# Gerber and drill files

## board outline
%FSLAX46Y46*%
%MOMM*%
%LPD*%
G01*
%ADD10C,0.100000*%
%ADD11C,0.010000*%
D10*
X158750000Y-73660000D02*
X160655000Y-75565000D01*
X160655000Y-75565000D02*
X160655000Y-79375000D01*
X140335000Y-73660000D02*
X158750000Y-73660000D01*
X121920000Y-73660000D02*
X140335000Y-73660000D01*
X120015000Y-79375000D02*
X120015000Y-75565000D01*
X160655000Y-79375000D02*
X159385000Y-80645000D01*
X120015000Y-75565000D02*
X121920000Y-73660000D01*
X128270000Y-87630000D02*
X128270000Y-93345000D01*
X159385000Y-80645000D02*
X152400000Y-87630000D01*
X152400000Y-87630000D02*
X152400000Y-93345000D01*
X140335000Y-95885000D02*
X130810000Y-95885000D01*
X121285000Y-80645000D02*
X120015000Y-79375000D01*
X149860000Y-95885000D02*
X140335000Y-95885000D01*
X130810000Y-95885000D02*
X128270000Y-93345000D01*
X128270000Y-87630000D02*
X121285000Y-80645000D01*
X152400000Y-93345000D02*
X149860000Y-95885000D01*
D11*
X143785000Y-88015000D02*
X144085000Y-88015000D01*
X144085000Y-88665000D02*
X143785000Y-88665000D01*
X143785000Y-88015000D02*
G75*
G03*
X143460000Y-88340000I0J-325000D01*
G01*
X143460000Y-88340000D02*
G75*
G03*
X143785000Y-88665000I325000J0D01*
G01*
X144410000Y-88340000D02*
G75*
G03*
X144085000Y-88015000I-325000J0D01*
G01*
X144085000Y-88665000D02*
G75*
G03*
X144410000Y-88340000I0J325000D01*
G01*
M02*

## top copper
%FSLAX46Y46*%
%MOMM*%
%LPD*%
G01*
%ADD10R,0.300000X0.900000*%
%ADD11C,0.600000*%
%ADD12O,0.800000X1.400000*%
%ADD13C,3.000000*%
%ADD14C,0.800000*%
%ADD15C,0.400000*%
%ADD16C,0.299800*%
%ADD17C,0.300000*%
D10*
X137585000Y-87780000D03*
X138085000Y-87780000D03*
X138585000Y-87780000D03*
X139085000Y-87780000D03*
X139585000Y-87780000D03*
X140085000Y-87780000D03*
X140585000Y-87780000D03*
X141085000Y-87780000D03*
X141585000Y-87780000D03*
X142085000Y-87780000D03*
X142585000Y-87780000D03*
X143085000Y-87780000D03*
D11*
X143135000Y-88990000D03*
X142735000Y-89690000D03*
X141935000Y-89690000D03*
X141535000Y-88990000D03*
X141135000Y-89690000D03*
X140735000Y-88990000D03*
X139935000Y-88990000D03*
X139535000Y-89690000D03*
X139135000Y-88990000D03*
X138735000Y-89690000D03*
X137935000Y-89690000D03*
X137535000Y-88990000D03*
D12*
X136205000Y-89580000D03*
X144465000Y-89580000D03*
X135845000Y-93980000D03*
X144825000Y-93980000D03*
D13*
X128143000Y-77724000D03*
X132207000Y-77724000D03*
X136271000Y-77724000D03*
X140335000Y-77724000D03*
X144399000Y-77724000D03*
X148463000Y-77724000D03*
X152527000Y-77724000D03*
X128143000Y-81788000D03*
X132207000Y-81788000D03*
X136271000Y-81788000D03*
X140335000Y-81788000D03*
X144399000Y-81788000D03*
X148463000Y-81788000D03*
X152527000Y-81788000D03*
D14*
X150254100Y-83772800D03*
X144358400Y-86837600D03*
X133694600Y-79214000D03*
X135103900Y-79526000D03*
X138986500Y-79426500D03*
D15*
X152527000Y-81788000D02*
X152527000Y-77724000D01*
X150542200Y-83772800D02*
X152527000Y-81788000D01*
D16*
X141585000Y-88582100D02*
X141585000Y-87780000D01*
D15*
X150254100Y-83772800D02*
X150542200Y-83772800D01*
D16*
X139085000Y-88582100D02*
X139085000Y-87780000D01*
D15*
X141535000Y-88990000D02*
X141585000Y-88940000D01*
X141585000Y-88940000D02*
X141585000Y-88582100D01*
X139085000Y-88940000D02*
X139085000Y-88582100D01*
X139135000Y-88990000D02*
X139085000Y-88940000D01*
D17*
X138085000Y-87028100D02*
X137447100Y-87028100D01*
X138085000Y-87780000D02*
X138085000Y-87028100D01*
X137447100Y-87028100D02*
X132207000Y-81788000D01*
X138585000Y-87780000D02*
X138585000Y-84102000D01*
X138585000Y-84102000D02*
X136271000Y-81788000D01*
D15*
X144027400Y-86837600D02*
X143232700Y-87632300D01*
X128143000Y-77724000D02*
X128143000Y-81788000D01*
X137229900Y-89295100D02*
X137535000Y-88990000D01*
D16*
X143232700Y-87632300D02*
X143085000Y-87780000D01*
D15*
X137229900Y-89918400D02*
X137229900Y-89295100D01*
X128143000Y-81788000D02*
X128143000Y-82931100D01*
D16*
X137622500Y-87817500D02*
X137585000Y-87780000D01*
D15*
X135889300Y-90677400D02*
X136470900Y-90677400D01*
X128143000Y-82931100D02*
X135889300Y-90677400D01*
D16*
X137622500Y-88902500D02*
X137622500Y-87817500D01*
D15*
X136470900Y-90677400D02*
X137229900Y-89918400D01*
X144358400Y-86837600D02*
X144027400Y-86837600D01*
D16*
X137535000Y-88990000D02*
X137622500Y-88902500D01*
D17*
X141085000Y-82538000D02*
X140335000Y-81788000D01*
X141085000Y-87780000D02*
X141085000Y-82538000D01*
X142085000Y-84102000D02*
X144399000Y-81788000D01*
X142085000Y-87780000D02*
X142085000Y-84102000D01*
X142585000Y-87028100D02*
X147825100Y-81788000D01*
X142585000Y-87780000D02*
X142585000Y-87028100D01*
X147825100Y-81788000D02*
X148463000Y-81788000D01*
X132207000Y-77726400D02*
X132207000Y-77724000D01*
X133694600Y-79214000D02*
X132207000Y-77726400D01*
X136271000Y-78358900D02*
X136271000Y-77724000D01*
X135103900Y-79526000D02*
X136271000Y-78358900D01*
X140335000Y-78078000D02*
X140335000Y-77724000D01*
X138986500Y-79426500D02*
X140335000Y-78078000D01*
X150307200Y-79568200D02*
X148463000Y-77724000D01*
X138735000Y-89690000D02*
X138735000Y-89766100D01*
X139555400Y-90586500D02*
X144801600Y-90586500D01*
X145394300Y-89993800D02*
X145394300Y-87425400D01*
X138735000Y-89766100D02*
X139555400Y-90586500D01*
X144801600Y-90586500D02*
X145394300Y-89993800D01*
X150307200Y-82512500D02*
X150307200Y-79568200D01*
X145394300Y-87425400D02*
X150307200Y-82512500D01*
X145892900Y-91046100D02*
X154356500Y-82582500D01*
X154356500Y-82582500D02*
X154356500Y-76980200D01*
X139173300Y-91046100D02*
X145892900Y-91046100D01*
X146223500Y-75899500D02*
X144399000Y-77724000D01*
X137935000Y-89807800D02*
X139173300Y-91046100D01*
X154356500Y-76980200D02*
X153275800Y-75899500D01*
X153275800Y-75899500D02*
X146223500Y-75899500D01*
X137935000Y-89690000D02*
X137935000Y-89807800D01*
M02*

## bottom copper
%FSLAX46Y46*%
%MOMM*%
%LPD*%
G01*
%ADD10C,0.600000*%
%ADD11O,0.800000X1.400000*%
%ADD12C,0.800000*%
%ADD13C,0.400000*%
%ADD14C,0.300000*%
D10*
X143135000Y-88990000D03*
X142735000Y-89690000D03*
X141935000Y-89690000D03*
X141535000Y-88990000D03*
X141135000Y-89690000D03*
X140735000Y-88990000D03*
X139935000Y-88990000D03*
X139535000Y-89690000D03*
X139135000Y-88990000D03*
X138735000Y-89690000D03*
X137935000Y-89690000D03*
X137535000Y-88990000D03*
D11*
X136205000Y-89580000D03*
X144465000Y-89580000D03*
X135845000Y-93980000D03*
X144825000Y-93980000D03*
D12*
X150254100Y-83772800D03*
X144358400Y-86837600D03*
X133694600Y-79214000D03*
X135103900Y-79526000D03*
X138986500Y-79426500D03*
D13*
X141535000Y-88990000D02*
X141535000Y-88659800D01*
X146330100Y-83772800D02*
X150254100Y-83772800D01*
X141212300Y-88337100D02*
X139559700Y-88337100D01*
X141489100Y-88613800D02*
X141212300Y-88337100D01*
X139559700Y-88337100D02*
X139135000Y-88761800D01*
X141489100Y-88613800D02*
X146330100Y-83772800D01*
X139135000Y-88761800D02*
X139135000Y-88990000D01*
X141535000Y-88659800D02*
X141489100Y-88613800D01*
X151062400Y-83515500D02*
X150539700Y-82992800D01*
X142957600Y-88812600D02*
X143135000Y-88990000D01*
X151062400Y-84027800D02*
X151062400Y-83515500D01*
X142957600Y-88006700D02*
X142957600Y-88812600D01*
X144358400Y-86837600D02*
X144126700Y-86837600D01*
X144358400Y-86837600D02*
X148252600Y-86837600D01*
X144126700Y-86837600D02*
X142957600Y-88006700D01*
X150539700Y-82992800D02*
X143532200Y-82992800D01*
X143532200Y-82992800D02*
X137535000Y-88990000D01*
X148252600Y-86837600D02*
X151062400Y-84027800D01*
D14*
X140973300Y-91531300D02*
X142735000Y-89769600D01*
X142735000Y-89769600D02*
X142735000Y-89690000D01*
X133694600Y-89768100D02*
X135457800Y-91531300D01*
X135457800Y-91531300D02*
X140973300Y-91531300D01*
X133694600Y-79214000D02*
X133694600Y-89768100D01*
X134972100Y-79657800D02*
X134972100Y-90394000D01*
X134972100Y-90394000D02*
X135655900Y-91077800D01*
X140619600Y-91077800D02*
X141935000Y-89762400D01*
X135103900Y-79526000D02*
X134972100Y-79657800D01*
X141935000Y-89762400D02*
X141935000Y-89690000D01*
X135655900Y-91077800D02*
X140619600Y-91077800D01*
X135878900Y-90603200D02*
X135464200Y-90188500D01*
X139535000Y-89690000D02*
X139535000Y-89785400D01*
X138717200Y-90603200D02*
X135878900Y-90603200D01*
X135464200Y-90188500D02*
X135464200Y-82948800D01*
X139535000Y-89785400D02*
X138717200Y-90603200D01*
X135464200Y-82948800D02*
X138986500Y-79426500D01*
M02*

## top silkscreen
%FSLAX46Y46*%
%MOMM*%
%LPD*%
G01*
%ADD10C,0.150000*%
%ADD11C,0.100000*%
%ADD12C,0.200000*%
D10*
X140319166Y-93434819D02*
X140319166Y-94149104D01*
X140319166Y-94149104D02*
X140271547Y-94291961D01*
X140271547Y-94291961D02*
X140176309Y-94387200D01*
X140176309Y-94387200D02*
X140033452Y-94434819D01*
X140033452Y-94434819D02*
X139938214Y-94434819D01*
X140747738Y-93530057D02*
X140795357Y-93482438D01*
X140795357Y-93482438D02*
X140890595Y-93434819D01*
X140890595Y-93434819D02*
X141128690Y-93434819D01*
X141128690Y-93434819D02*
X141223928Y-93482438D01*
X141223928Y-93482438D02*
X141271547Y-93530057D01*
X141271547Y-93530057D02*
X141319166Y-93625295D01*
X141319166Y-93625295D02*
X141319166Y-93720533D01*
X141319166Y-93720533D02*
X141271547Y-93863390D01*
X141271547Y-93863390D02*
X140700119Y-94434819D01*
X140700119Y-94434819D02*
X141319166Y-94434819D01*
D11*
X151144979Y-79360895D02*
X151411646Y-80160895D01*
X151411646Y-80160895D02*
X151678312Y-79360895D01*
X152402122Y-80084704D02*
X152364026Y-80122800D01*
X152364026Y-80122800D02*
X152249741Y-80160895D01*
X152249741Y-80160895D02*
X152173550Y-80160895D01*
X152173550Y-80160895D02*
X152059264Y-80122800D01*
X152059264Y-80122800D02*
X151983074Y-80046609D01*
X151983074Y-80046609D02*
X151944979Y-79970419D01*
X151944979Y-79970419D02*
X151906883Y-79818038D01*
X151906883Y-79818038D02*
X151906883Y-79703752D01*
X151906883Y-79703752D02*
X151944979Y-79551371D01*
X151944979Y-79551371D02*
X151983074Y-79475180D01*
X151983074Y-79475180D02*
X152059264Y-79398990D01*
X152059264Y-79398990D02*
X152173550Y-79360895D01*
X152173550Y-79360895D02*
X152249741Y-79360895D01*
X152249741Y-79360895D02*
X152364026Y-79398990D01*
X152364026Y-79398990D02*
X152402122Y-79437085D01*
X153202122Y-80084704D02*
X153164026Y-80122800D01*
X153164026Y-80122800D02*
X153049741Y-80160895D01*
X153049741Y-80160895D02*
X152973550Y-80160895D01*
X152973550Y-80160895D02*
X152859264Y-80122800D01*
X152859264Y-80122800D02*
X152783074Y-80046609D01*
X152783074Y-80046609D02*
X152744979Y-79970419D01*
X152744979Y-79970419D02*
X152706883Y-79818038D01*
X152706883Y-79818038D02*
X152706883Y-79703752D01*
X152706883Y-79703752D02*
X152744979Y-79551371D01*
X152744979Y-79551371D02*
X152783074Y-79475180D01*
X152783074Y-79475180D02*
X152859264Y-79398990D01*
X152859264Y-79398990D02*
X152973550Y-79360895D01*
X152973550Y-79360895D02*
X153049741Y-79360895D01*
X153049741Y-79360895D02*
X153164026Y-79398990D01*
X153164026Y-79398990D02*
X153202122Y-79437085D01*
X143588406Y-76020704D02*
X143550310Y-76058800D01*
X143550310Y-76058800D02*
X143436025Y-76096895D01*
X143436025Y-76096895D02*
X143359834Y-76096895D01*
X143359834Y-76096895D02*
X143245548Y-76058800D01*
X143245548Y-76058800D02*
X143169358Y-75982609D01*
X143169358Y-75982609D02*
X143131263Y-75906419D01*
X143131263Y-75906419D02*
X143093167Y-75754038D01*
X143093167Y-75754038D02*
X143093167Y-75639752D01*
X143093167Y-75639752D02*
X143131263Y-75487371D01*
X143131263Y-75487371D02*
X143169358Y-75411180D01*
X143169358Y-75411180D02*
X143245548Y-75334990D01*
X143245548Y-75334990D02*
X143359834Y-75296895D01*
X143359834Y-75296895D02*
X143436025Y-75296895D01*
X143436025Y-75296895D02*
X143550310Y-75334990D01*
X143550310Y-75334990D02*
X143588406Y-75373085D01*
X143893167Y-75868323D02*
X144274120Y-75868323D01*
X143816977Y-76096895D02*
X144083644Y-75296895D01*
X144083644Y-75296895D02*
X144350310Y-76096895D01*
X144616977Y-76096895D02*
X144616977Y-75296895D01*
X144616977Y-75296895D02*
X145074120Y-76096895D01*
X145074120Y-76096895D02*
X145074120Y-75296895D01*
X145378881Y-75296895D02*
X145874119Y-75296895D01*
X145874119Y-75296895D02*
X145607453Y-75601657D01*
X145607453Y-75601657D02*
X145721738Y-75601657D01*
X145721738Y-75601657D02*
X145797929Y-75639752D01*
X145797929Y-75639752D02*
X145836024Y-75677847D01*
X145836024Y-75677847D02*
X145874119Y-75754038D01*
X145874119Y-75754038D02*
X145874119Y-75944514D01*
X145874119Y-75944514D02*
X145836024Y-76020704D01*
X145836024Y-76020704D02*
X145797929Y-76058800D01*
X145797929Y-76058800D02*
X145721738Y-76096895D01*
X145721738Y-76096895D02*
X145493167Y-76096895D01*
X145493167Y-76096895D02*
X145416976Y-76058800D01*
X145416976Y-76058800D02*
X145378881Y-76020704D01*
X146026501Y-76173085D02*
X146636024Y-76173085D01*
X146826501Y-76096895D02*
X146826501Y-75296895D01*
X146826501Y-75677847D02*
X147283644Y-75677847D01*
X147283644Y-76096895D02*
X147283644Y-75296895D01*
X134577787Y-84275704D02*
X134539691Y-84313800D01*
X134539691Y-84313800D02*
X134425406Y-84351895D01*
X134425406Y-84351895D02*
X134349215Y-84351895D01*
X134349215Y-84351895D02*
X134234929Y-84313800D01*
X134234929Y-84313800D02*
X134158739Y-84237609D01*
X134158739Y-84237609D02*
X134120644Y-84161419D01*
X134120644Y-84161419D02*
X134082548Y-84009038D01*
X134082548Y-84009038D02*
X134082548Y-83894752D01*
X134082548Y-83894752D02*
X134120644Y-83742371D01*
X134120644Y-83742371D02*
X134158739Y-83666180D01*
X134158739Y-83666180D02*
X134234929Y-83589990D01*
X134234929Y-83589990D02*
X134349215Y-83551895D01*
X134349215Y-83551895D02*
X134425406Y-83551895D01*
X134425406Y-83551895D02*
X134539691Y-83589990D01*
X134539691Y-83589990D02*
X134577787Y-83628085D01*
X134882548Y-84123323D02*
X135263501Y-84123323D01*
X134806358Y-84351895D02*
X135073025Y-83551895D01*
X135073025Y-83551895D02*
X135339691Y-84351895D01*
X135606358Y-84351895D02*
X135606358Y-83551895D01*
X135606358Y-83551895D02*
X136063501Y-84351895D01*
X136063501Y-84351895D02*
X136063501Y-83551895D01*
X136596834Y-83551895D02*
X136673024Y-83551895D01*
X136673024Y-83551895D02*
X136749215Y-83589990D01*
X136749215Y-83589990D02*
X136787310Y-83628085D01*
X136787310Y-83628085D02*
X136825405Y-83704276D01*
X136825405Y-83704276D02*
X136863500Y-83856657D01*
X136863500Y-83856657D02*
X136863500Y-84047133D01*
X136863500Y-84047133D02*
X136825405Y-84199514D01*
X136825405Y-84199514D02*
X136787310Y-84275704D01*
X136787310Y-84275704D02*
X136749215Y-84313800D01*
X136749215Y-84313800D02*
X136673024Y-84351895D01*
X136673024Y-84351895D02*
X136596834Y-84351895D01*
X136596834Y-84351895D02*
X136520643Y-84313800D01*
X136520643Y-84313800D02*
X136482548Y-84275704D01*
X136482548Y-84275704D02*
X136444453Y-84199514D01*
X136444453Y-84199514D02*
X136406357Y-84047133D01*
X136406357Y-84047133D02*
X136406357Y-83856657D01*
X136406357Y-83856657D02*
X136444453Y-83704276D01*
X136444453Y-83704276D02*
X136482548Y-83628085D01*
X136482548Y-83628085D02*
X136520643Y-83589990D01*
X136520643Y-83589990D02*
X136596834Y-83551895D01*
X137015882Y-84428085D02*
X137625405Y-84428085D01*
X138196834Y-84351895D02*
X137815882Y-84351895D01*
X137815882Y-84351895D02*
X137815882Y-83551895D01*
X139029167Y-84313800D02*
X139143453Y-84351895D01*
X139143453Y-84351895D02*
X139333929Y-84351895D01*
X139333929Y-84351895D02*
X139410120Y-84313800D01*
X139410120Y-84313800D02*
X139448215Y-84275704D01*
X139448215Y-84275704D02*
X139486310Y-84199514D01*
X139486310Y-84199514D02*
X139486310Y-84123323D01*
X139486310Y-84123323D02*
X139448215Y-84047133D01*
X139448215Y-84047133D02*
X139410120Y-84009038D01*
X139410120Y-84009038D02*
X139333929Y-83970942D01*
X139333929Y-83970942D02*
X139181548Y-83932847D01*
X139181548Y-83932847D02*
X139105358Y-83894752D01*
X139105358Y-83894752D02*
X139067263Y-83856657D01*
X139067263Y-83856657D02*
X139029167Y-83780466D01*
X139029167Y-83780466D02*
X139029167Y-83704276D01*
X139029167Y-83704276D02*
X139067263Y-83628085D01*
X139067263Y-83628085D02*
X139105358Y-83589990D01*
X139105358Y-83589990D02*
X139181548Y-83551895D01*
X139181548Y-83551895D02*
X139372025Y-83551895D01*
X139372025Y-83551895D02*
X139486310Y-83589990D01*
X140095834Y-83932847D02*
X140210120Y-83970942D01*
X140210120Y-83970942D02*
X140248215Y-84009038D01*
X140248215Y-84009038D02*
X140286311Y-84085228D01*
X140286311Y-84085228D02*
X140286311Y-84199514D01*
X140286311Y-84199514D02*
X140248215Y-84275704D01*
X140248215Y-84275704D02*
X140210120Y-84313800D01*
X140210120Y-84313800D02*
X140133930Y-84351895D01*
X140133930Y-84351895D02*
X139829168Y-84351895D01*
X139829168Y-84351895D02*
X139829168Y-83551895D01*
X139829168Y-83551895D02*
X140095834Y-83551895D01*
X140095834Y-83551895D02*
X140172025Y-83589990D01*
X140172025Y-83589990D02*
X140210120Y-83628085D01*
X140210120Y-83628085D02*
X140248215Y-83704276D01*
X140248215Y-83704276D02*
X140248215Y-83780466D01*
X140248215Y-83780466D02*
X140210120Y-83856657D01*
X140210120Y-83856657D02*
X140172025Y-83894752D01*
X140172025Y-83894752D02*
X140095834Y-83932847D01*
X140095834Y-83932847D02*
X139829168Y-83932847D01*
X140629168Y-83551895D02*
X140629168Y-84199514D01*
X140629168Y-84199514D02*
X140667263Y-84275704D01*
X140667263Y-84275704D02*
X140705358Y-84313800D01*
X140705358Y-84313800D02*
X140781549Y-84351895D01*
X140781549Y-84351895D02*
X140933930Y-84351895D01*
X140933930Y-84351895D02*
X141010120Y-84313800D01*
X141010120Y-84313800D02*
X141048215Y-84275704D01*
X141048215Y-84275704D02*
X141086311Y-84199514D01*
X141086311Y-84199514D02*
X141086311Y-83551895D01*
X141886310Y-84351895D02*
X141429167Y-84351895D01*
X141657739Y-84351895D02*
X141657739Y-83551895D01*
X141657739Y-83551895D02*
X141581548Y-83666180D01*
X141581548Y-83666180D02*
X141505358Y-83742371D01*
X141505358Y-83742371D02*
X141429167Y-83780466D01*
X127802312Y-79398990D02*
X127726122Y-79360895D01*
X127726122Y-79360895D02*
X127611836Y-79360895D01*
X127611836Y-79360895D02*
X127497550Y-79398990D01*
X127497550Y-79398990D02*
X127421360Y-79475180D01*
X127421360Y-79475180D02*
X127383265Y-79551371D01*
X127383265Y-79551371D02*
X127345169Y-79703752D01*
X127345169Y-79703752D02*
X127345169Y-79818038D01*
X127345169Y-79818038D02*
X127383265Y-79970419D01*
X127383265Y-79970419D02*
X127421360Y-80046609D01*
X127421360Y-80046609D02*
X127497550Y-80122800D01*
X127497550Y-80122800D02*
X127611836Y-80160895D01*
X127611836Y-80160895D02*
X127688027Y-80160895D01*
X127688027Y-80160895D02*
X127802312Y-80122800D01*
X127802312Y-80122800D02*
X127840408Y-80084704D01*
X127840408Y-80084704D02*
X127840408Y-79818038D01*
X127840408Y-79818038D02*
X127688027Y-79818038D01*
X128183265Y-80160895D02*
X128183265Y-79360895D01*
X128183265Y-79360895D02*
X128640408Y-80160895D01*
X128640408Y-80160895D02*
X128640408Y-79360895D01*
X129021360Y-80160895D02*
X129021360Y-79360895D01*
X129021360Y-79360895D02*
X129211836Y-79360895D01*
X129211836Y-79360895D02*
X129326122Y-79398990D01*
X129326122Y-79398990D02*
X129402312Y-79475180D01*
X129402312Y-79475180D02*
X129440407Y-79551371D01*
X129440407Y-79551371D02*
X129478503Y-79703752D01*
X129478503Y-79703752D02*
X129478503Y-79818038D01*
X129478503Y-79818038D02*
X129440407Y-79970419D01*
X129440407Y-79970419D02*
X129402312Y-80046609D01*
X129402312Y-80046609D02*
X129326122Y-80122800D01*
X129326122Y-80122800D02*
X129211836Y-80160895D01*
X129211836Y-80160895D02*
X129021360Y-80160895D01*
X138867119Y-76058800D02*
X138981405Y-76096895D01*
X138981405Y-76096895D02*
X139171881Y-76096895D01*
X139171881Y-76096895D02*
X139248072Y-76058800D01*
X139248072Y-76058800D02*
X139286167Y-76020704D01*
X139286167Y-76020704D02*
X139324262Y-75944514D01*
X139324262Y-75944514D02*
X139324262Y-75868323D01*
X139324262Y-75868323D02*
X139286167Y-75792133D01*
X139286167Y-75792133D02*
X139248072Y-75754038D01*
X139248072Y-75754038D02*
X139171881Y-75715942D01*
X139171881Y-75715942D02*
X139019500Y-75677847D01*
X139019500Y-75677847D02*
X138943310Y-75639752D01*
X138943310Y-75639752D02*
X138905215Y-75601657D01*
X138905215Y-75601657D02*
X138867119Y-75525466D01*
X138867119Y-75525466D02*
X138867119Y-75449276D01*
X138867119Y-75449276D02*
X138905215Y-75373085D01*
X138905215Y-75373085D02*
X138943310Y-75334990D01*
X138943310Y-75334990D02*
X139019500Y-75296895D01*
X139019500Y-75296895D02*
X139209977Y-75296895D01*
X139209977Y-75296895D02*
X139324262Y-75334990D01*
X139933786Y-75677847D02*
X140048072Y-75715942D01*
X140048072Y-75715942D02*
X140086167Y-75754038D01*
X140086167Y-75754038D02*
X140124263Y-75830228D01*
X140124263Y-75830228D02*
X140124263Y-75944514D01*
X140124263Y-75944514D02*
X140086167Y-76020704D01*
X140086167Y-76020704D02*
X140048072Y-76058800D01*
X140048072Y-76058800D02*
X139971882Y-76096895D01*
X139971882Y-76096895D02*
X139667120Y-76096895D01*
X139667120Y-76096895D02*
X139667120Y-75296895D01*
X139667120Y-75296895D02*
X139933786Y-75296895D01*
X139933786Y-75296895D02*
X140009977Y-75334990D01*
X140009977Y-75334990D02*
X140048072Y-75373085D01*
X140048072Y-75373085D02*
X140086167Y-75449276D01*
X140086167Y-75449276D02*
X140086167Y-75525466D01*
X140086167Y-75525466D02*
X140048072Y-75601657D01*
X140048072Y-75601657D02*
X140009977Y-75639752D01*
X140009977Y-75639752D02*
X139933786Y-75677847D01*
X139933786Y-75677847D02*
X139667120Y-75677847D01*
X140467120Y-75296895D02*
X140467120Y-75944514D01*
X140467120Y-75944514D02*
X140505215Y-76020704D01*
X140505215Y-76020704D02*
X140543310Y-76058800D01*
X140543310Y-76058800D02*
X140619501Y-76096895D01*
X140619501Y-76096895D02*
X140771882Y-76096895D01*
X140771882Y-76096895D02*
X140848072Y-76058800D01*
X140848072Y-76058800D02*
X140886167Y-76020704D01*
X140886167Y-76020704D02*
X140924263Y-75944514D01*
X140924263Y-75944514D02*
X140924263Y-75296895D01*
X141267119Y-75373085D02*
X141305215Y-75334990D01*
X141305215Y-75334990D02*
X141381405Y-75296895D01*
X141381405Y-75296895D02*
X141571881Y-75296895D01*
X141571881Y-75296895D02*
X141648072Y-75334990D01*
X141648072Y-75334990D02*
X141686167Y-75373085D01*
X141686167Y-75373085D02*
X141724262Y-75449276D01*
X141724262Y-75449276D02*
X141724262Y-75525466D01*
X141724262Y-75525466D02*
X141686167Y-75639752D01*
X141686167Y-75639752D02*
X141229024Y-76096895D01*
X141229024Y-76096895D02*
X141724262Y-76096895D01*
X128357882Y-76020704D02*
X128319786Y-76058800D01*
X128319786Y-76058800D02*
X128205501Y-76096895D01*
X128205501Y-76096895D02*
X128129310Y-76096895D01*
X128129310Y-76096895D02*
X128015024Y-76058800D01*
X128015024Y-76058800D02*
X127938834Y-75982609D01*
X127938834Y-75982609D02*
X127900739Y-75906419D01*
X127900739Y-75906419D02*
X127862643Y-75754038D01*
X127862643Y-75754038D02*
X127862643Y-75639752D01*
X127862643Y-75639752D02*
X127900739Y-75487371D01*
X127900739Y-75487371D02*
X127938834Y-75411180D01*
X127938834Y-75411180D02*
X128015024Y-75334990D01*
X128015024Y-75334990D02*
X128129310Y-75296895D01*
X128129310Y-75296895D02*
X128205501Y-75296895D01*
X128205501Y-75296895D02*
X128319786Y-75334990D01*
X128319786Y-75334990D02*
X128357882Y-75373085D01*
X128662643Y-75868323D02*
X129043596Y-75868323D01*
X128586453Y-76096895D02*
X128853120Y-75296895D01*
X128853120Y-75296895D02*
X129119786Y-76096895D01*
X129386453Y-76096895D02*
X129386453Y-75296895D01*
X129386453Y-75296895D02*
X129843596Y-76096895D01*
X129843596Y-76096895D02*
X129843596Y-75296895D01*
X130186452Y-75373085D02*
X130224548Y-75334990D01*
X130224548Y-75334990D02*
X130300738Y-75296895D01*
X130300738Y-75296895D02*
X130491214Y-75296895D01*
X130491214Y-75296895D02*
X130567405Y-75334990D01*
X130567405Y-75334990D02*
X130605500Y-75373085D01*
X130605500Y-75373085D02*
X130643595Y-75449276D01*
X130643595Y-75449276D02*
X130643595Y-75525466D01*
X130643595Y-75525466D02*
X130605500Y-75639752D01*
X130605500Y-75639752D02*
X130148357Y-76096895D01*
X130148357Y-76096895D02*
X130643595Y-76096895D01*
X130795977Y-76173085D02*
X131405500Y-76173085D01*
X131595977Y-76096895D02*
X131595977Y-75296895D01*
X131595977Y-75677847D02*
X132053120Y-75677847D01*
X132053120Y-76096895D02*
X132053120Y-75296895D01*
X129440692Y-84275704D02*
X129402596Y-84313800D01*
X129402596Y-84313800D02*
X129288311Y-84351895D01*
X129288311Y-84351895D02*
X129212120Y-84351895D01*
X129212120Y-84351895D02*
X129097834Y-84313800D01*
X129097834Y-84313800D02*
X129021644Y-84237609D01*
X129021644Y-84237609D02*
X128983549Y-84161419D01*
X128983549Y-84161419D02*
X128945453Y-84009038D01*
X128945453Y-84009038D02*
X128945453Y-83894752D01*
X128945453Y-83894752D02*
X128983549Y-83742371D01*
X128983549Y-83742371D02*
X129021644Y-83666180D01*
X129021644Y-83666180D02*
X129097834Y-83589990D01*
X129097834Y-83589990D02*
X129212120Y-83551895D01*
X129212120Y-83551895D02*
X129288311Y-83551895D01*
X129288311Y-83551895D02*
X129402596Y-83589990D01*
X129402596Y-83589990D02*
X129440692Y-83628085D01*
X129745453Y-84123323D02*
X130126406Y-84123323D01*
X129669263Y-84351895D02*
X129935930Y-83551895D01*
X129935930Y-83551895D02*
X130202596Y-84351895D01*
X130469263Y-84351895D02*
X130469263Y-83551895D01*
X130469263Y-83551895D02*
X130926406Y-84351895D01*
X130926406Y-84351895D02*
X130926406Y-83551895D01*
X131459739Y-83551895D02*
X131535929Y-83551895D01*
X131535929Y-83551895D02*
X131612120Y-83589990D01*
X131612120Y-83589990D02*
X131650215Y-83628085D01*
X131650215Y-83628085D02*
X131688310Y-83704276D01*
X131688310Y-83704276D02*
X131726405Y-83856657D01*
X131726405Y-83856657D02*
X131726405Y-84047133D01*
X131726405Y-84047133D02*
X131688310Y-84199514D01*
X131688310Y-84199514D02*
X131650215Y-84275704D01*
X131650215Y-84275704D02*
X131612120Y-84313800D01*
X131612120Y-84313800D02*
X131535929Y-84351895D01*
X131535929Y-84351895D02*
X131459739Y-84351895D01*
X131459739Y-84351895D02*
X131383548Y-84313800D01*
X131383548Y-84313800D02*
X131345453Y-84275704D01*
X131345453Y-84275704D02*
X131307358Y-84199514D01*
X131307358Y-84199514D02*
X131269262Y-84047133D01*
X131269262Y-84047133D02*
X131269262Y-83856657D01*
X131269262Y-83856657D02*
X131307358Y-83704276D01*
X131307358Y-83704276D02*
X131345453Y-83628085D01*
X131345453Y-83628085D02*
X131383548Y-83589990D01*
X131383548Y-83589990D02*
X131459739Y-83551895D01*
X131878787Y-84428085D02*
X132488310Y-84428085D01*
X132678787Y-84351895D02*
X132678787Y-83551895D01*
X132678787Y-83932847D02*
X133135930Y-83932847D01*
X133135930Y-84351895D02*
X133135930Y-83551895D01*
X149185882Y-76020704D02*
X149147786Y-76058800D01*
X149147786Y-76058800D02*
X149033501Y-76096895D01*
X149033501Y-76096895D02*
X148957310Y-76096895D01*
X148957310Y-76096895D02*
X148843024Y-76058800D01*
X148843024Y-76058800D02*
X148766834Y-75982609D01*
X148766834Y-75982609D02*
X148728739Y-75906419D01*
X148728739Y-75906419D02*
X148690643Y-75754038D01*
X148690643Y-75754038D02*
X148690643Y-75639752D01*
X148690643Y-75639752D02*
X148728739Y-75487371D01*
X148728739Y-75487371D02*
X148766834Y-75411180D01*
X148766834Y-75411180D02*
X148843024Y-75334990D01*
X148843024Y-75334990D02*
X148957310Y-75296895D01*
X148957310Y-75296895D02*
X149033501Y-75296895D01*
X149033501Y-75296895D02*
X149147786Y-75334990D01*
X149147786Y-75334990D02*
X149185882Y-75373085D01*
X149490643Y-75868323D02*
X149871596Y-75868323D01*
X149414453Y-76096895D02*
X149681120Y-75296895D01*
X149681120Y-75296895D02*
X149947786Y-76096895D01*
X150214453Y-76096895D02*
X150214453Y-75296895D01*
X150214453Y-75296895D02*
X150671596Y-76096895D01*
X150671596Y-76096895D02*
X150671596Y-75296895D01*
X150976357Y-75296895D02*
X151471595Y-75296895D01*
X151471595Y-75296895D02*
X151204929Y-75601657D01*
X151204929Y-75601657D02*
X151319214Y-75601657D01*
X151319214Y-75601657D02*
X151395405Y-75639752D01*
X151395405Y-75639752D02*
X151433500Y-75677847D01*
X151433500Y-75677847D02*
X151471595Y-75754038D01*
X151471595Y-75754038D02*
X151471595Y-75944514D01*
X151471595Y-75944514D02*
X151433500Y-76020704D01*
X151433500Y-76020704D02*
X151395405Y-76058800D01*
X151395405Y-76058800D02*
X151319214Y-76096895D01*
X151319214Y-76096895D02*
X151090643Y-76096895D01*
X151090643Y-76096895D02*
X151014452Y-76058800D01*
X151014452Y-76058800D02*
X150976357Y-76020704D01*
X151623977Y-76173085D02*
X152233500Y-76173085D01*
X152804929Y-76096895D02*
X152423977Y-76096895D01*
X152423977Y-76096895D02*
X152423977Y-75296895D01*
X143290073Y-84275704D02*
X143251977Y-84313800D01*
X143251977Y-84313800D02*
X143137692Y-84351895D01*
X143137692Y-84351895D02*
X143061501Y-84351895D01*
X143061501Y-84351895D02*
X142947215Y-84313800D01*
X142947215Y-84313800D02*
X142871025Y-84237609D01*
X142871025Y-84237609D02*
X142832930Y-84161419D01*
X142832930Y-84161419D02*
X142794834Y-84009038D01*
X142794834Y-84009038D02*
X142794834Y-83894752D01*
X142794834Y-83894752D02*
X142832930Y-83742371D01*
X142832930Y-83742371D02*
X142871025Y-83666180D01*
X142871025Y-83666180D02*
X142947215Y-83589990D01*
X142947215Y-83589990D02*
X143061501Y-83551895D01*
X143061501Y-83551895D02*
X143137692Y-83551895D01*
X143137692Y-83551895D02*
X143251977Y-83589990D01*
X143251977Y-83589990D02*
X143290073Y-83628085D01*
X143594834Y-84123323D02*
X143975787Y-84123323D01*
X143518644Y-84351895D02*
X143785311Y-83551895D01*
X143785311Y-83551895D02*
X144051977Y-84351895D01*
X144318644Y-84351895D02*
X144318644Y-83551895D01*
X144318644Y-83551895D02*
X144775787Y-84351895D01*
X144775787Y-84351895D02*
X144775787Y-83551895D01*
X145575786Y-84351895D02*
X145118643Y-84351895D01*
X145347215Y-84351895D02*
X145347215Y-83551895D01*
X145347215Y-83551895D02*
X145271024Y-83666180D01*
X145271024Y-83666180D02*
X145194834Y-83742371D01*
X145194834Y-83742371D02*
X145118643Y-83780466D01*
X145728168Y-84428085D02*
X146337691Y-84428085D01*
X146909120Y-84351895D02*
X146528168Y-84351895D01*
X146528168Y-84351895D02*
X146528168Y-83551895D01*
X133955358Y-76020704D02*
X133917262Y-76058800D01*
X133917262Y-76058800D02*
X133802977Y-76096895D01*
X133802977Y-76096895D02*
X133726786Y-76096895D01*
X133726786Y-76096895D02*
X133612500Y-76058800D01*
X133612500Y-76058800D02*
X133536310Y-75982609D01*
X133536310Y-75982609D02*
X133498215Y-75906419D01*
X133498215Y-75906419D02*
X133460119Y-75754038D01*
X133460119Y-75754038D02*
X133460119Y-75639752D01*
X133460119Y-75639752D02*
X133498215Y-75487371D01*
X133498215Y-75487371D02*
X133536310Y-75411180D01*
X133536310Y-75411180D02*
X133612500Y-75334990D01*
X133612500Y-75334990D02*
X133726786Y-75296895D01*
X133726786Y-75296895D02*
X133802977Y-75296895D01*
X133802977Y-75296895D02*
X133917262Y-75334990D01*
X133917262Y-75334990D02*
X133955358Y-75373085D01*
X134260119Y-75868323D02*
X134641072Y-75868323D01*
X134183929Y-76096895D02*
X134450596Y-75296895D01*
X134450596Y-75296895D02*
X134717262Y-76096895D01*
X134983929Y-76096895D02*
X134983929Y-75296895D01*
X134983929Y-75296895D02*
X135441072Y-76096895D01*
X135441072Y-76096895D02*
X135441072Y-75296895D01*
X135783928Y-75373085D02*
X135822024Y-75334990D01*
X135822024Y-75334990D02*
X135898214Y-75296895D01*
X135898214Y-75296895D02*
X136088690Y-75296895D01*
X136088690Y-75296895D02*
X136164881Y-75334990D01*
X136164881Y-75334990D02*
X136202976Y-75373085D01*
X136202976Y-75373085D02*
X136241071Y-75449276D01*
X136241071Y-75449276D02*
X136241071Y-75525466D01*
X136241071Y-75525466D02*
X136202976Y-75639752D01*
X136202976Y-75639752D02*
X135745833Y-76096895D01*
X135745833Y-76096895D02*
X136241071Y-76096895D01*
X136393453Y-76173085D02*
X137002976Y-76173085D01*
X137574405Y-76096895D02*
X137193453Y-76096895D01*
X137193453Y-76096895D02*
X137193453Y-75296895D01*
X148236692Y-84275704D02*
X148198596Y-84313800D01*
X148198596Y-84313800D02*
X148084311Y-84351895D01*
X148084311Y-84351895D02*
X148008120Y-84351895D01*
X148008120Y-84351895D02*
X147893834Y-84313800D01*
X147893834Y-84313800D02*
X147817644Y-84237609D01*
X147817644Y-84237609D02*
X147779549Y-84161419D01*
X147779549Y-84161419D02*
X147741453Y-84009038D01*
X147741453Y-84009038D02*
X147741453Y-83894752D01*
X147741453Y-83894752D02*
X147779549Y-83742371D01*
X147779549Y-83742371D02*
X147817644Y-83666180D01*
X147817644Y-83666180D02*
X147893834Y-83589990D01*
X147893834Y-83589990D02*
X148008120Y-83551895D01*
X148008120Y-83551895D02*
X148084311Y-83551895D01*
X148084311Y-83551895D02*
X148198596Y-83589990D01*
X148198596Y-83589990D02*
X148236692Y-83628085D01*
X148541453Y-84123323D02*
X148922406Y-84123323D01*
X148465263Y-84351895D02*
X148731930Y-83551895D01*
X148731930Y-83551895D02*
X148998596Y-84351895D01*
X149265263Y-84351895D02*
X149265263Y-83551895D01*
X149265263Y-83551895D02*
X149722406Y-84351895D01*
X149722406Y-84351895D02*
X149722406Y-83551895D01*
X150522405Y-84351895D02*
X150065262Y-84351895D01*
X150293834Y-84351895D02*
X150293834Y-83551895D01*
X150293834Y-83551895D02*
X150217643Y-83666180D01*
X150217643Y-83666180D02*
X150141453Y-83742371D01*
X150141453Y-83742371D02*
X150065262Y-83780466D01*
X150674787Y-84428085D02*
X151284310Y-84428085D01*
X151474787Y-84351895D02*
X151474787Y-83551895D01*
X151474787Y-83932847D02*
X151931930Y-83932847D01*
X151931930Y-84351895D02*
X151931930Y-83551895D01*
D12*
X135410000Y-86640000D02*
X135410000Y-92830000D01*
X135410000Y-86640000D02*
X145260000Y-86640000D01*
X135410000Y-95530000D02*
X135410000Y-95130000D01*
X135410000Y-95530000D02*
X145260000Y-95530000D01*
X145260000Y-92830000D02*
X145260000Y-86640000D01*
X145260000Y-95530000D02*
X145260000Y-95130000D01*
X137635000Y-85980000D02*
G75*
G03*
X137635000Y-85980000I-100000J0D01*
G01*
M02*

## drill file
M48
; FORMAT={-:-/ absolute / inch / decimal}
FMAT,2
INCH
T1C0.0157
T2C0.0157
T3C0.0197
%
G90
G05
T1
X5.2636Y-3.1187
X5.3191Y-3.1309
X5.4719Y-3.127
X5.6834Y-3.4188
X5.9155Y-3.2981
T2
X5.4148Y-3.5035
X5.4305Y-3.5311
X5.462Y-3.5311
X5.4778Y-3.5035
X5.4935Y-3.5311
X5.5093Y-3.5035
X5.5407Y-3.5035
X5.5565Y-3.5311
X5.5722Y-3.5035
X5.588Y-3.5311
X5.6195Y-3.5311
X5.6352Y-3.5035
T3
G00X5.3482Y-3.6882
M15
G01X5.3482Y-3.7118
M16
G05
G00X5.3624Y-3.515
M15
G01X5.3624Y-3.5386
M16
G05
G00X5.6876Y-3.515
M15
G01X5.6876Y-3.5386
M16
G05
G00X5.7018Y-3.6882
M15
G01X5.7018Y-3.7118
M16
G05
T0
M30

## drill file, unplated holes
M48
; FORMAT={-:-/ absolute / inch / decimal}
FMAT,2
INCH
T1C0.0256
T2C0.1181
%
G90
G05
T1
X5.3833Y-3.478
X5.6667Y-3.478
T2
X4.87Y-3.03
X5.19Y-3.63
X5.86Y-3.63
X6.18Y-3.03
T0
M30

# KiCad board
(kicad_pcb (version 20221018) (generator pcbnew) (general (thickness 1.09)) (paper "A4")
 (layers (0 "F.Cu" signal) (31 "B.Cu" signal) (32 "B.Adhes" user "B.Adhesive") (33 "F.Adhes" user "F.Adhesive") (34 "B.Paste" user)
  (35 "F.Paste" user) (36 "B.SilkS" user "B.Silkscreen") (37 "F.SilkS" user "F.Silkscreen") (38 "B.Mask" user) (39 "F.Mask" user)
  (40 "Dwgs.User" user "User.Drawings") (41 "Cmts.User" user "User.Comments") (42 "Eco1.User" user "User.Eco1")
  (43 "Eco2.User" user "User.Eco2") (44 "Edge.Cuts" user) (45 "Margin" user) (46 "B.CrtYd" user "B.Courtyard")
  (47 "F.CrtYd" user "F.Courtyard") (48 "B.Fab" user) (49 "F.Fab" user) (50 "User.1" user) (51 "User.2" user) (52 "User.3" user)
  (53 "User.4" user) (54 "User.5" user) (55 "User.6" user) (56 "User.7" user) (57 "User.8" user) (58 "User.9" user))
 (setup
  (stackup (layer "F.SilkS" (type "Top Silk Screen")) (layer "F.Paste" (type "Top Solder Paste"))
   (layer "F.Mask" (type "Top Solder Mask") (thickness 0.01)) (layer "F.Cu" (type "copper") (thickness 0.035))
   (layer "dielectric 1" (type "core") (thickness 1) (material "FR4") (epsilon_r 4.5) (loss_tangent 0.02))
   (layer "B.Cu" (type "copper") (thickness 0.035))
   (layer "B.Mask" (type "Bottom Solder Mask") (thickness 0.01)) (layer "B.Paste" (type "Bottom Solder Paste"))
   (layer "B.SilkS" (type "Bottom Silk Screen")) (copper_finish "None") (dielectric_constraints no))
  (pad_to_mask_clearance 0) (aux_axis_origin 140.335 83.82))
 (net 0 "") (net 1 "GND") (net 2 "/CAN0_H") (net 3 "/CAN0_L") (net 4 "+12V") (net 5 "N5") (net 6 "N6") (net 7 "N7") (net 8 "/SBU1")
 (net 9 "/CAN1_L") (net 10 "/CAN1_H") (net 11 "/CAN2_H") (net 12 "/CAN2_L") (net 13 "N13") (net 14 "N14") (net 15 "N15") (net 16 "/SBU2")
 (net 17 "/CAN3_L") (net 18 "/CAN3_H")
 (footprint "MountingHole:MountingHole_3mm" (layer "F.Cu") (at 123.698 76.962)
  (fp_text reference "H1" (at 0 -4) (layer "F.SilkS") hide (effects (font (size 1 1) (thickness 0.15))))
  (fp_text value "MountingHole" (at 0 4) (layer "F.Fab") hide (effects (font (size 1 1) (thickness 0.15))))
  (pad "" np_thru_hole circle (at 0 0) (size 3 3) (drill 3) (layers "*.Cu" "*.Mask")))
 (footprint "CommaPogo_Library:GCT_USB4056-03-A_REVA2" (layer "F.Cu") (at 140.335 93.98) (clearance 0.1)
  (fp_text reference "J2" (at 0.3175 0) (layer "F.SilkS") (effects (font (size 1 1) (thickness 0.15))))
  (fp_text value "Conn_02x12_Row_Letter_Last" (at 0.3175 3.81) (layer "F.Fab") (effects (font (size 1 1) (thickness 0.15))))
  (fp_line (start -4.925 -7.34) (end -4.925 -1.15) (stroke (width 0.2) (type solid)) (layer "F.SilkS"))
  (fp_line (start -4.925 -7.34) (end 4.925 -7.34) (stroke (width 0.2) (type solid)) (layer "F.SilkS"))
  (fp_line (start -4.925 1.55) (end -4.925 1.15) (stroke (width 0.2) (type solid)) (layer "F.SilkS"))
  (fp_line (start -4.925 1.55) (end 4.925 1.55) (stroke (width 0.2) (type solid)) (layer "F.SilkS"))
  (fp_line (start 4.925 -1.15) (end 4.925 -7.34) (stroke (width 0.2) (type solid)) (layer "F.SilkS"))
  (fp_line (start 4.925 1.55) (end 4.925 1.15) (stroke (width 0.2) (type solid)) (layer "F.SilkS"))
  (fp_circle (center -2.8 -8) (end -2.7 -8) (stroke (width 0.2) (type solid)) (fill none) (layer "F.SilkS"))
  (fp_line (start 3.45 -5.965) (end 3.75 -5.965) (stroke (width 0.01) (type solid)) (layer "Edge.Cuts"))
  (fp_line (start 3.75 -5.315) (end 3.45 -5.315) (stroke (width 0.01) (type solid)) (layer "Edge.Cuts"))
  (fp_arc (start 3.125 -5.64) (mid 3.22019 -5.86981) (end 3.45 -5.965) (stroke (width 0.01) (type solid)) (layer "Edge.Cuts"))
  (fp_arc (start 3.45 -5.315) (mid 3.22019 -5.41019) (end 3.125 -5.64) (stroke (width 0.01) (type solid)) (layer "Edge.Cuts"))
  (fp_arc (start 3.75 -5.965) (mid 3.97981 -5.86981) (end 4.075 -5.64) (stroke (width 0.01) (type solid)) (layer "Edge.Cuts"))
  (fp_arc (start 4.075 -5.64) (mid 3.97981 -5.41019) (end 3.75 -5.315) (stroke (width 0.01) (type solid)) (layer "Edge.Cuts"))
  (pad "" np_thru_hole circle (at -3.6 -5.64) (size 0.65 0.65) (drill 0.65) (layers "*.Cu" "*.Mask"))
  (pad "" np_thru_hole circle (at 3.6 -5.64) (size 0.65 0.65) (drill 0.65) (layers "*.Cu" "*.Mask"))
  (pad "A1" smd rect (at -2.75 -6.2) (size 0.3 0.9) (layers "F.Cu" "F.Paste" "F.Mask") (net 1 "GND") (solder_mask_margin 0.102))
  (pad "A2" smd rect (at -2.25 -6.2) (size 0.3 0.9) (layers "F.Cu" "F.Paste" "F.Mask") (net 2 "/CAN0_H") (solder_mask_margin 0.102))
  (pad "A3" smd rect (at -1.75 -6.2) (size 0.3 0.9) (layers "F.Cu" "F.Paste" "F.Mask") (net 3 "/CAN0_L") (solder_mask_margin 0.102))
  (pad "A4" smd rect (at -1.25 -6.2) (size 0.3 0.9) (layers "F.Cu" "F.Paste" "F.Mask") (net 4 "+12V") (solder_mask_margin 0.102))
  (pad "A5" smd rect (at -0.75 -6.2) (size 0.3 0.9) (layers "F.Cu" "F.Paste" "F.Mask") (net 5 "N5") (solder_mask_margin 0.102))
  (pad "A6" smd rect (at -0.25 -6.2) (size 0.3 0.9) (layers "F.Cu" "F.Paste" "F.Mask") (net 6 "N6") (solder_mask_margin 0.102))
  (pad "A7" smd rect (at 0.25 -6.2) (size 0.3 0.9) (layers "F.Cu" "F.Paste" "F.Mask") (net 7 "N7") (solder_mask_margin 0.102))
  (pad "A8" smd rect (at 0.75 -6.2) (size 0.3 0.9) (layers "F.Cu" "F.Paste" "F.Mask") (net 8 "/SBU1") (solder_mask_margin 0.102))
  (pad "A9" smd rect (at 1.25 -6.2) (size 0.3 0.9) (layers "F.Cu" "F.Paste" "F.Mask") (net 4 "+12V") (solder_mask_margin 0.102))
  (pad "A10" smd rect (at 1.75 -6.2) (size 0.3 0.9) (layers "F.Cu" "F.Paste" "F.Mask") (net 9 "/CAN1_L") (solder_mask_margin 0.102))
  (pad "A11" smd rect (at 2.25 -6.2) (size 0.3 0.9) (layers "F.Cu" "F.Paste" "F.Mask") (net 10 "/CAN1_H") (solder_mask_margin 0.102))
  (pad "A12" smd rect (at 2.75 -6.2) (size 0.3 0.9) (layers "F.Cu" "F.Paste" "F.Mask") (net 1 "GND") (solder_mask_margin 0.102))
  (pad "B1" thru_hole circle (at 2.8 -4.99) (size 0.6 0.6) (drill 0.4) (layers "*.Cu" "*.Mask") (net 1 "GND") (solder_mask_margin 0.102))
  (pad "B2" thru_hole circle (at 2.4 -4.29) (size 0.6 0.6) (drill 0.4) (layers "*.Cu" "*.Mask") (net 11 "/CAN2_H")
   (solder_mask_margin 0.102))
  (pad "B3" thru_hole circle (at 1.6 -4.29) (size 0.6 0.6) (drill 0.4) (layers "*.Cu" "*.Mask") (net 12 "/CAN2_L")
   (solder_mask_margin 0.102))
  (pad "B4" thru_hole circle (at 1.2 -4.99) (size 0.6 0.6) (drill 0.4) (layers "*.Cu" "*.Mask") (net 4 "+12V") (solder_mask_margin 0.102))
  (pad "B5" thru_hole circle (at 0.8 -4.29) (size 0.6 0.6) (drill 0.4) (layers "*.Cu" "*.Mask") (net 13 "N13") (solder_mask_margin 0.102))
  (pad "B6" thru_hole circle (at 0.4 -4.99) (size 0.6 0.6) (drill 0.4) (layers "*.Cu" "*.Mask") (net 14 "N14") (solder_mask_margin 0.102))
  (pad "B7" thru_hole circle (at -0.4 -4.99) (size 0.6 0.6) (drill 0.4) (layers "*.Cu" "*.Mask") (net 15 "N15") (solder_mask_margin 0.102))
  (pad "B8" thru_hole circle (at -0.8 -4.29) (size 0.6 0.6) (drill 0.4) (layers "*.Cu" "*.Mask") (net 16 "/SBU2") (solder_mask_margin 0.102))
  (pad "B9" thru_hole circle (at -1.2 -4.99) (size 0.6 0.6) (drill 0.4) (layers "*.Cu" "*.Mask") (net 4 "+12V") (solder_mask_margin 0.102))
  (pad "B10" thru_hole circle (at -1.6 -4.29) (size 0.6 0.6) (drill 0.4) (layers "*.Cu" "*.Mask") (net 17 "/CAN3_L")
   (solder_mask_margin 0.102))
  (pad "B11" thru_hole circle (at -2.4 -4.29) (size 0.6 0.6) (drill 0.4) (layers "*.Cu" "*.Mask") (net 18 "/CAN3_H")
   (solder_mask_margin 0.102))
  (pad "B12" thru_hole circle (at -2.8 -4.99) (size 0.6 0.6) (drill 0.4) (layers "*.Cu" "*.Mask") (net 1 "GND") (solder_mask_margin 0.102))
  (pad "S1" thru_hole oval (at -4.13 -4.4) (size 0.8 1.4) (drill oval 0.5 1.1) (layers "*.Cu" "*.Mask") (solder_mask_margin 0.102))
  (pad "S2" thru_hole oval (at 4.13 -4.4) (size 0.8 1.4) (drill oval 0.5 1.1) (layers "*.Cu" "*.Mask") (solder_mask_margin 0.102))
  (pad "S3" thru_hole oval (at -4.49 0) (size 0.8 1.4) (drill oval 0.5 1.1) (layers "*.Cu" "*.Mask") (solder_mask_margin 0.102))
  (pad "S4" thru_hole oval (at 4.49 0) (size 0.8 1.4) (drill oval 0.5 1.1) (layers "*.Cu" "*.Mask") (solder_mask_margin 0.102)))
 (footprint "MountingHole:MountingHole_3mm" (layer "F.Cu") (at 148.844 92.202)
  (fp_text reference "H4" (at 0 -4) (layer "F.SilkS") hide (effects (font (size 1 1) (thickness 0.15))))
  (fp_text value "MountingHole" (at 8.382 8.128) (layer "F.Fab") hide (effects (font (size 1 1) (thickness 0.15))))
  (pad "" np_thru_hole circle (at 0 0) (size 3 3) (drill 3) (layers "*.Cu" "*.Mask")))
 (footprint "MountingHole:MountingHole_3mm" (layer "F.Cu") (at 131.826 92.202)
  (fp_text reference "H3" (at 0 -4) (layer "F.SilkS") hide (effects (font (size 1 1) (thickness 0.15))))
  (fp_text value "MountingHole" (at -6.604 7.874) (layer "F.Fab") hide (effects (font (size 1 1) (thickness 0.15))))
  (pad "" np_thru_hole circle (at 0 0) (size 3 3) (drill 3) (layers "*.Cu" "*.Mask")))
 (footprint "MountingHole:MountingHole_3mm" (layer "F.Cu") (at 156.972 76.962)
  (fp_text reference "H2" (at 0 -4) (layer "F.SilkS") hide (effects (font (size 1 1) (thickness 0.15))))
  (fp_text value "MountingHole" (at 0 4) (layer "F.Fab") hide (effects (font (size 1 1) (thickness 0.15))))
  (pad "" np_thru_hole circle (at 0 0) (size 3 3) (drill 3) (layers "*.Cu" "*.Mask")))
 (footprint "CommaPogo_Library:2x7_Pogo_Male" (layer "F.Cu") (at 140.335 83.82)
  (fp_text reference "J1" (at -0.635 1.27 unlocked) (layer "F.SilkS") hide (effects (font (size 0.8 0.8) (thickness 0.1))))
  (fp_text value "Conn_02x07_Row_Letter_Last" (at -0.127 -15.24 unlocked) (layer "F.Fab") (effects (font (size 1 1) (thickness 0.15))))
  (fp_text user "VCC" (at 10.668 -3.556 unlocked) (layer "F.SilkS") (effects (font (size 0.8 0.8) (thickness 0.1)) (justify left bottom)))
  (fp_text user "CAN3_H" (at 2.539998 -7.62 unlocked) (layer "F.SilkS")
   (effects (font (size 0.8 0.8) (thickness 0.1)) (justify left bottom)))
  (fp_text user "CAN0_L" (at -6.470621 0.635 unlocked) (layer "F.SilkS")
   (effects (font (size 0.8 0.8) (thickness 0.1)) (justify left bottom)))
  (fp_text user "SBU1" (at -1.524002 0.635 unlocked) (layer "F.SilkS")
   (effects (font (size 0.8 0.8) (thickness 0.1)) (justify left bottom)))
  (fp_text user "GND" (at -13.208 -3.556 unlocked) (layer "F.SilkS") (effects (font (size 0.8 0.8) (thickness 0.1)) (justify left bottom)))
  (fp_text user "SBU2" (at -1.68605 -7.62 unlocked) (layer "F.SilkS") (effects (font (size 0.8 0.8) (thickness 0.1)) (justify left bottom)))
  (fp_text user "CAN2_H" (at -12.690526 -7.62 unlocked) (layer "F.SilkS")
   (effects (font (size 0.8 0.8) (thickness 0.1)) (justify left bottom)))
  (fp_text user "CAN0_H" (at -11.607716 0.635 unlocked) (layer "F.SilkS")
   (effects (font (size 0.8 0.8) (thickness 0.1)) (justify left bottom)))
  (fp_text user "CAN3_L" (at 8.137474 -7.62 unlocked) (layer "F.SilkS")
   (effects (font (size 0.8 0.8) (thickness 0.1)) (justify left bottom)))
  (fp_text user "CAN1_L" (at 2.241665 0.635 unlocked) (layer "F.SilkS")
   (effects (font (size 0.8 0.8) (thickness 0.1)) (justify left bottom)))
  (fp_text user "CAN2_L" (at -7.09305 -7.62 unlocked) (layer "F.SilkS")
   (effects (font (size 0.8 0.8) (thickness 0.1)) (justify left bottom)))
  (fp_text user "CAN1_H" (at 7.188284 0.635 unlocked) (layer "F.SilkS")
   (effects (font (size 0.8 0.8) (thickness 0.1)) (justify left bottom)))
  (pad "1" smd circle (at -12.192 -6.096) (size 3 3) (layers "F.Cu" "F.Paste" "F.Mask") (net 1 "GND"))
  (pad "2" smd circle (at -8.128 -6.096) (size 3 3) (layers "F.Cu" "F.Paste" "F.Mask") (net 11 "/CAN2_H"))
  (pad "3" smd circle (at -4.064 -6.096) (size 3 3) (layers "F.Cu" "F.Paste" "F.Mask") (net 12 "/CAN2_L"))
  (pad "4" smd circle (at 0 -6.096) (size 3 3) (layers "F.Cu" "F.Paste" "F.Mask") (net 16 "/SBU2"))
  (pad "5" smd circle (at 4.064 -6.096) (size 3 3) (layers "F.Cu" "F.Paste" "F.Mask") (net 18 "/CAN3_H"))
  (pad "6" smd circle (at 8.128 -6.096) (size 3 3) (layers "F.Cu" "F.Paste" "F.Mask") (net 17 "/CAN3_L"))
  (pad "7" smd circle (at 12.192 -6.096) (size 3 3) (layers "F.Cu" "F.Paste" "F.Mask") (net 4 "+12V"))
  (pad "8" smd circle (at -12.192 -2.032) (size 3 3) (layers "F.Cu" "F.Paste" "F.Mask") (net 1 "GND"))
  (pad "9" smd circle (at -8.128 -2.032) (size 3 3) (layers "F.Cu" "F.Paste" "F.Mask") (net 2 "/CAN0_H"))
  (pad "10" smd circle (at -4.064 -2.032) (size 3 3) (layers "F.Cu" "F.Paste" "F.Mask") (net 3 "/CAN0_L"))
  (pad "11" smd circle (at 0 -2.032) (size 3 3) (layers "F.Cu" "F.Paste" "F.Mask") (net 8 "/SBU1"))
  (pad "12" smd circle (at 4.064 -2.032) (size 3 3) (layers "F.Cu" "F.Paste" "F.Mask") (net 9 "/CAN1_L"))
  (pad "13" smd circle (at 8.128 -2.032) (size 3 3) (layers "F.Cu" "F.Paste" "F.Mask") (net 10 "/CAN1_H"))
  (pad "14" smd circle (at 12.192 -2.032) (size 3 3) (layers "F.Cu" "F.Paste" "F.Mask") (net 4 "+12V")))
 (gr_line (start 158.75 73.66) (end 160.655 75.565) (stroke (width 0.1) (type default)) (layer "Edge.Cuts"))
 (gr_line (start 160.655 75.565) (end 160.655 79.375) (stroke (width 0.1) (type default)) (layer "Edge.Cuts"))
 (gr_line (start 140.335 73.66) (end 158.75 73.66) (stroke (width 0.1) (type default)) (layer "Edge.Cuts"))
 (gr_line (start 121.92 73.66) (end 140.335 73.66) (stroke (width 0.1) (type default)) (layer "Edge.Cuts"))
 (gr_line (start 120.015 79.375) (end 120.015 75.565) (stroke (width 0.1) (type default)) (layer "Edge.Cuts"))
 (gr_line (start 160.655 79.375) (end 159.385 80.645) (stroke (width 0.1) (type default)) (layer "Edge.Cuts"))
 (gr_line (start 120.015 75.565) (end 121.92 73.66) (stroke (width 0.1) (type default)) (layer "Edge.Cuts"))
 (gr_line (start 128.27 87.63) (end 128.27 93.345) (stroke (width 0.1) (type default)) (layer "Edge.Cuts"))
 (gr_line (start 159.385 80.645) (end 152.4 87.63) (stroke (width 0.1) (type default)) (layer "Edge.Cuts"))
 (gr_line (start 152.4 87.63) (end 152.4 93.345) (stroke (width 0.1) (type default)) (layer "Edge.Cuts"))
 (gr_line (start 140.335 95.885) (end 130.81 95.885) (stroke (width 0.1) (type default)) (layer "Edge.Cuts"))
 (gr_line (start 121.285 80.645) (end 120.015 79.375) (stroke (width 0.1) (type default)) (layer "Edge.Cuts"))
 (gr_line (start 149.86 95.885) (end 140.335 95.885) (stroke (width 0.1) (type default)) (layer "Edge.Cuts"))
 (gr_line (start 130.81 95.885) (end 128.27 93.345) (stroke (width 0.1) (type default)) (layer "Edge.Cuts"))
 (gr_line (start 128.27 87.63) (end 121.285 80.645) (stroke (width 0.1) (type default)) (layer "Edge.Cuts"))
 (gr_line (start 152.4 93.345) (end 149.86 95.885) (stroke (width 0.1) (type default)) (layer "Edge.Cuts"))
 (segment (start 152.527 81.788) (end 152.527 77.724) (width 0.4) (layer "F.Cu") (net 4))
 (segment (start 150.5422 83.7728) (end 152.527 81.788) (width 0.4) (layer "F.Cu") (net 4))
 (segment (start 141.585 88.5821) (end 141.585 87.78) (width 0.2998) (layer "F.Cu") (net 4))
 (segment (start 150.2541 83.7728) (end 150.5422 83.7728) (width 0.4) (layer "F.Cu") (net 4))
 (segment (start 139.085 88.5821) (end 139.085 87.78) (width 0.2998) (layer "F.Cu") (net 4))
 (segment (start 141.535 88.99) (end 141.585 88.94) (width 0.4) (layer "F.Cu") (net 4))
 (segment (start 141.585 88.94) (end 141.585 88.5821) (width 0.4) (layer "F.Cu") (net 4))
 (segment (start 139.085 88.94) (end 139.085 88.5821) (width 0.4) (layer "F.Cu") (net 4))
 (segment (start 139.135 88.99) (end 139.085 88.94) (width 0.4) (layer "F.Cu") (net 4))
 (via (at 150.2541 83.7728) (size 0.8) (drill 0.4) (layers "F.Cu" "B.Cu") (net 4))
 (segment (start 141.535 88.99) (end 141.535 88.6598) (width 0.4) (layer "B.Cu") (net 4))
 (segment (start 146.3301 83.7728) (end 150.2541 83.7728) (width 0.4) (layer "B.Cu") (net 4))
 (segment (start 141.2123 88.3371) (end 139.5597 88.3371) (width 0.4) (layer "B.Cu") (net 4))
 (segment (start 141.4891 88.6138) (end 141.2123 88.3371) (width 0.4) (layer "B.Cu") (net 4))
 (segment (start 139.5597 88.3371) (end 139.135 88.7618) (width 0.4) (layer "B.Cu") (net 4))
 (segment (start 141.4891 88.6138) (end 146.3301 83.7728) (width 0.4) (layer "B.Cu") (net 4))
 (segment (start 139.135 88.7618) (end 139.135 88.99) (width 0.4) (layer "B.Cu") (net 4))
 (segment (start 141.535 88.6598) (end 141.4891 88.6138) (width 0.4) (layer "B.Cu") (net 4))
 (segment (start 138.085 87.0281) (end 137.4471 87.0281) (width 0.3) (layer "F.Cu") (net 2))
 (segment (start 138.085 87.78) (end 138.085 87.0281) (width 0.3) (layer "F.Cu") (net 2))
 (segment (start 137.4471 87.0281) (end 132.207 81.788) (width 0.3) (layer "F.Cu") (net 2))
 (segment (start 138.585 87.78) (end 138.585 84.102) (width 0.3) (layer "F.Cu") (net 3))
 (segment (start 138.585 84.102) (end 136.271 81.788) (width 0.3) (layer "F.Cu") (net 3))
 (segment (start 144.0274 86.8376) (end 143.2327 87.6323) (width 0.4) (layer "F.Cu") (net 1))
 (segment (start 128.143 77.724) (end 128.143 81.788) (width 0.4) (layer "F.Cu") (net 1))
 (segment (start 137.2299 89.2951) (end 137.535 88.99) (width 0.4) (layer "F.Cu") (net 1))
 (segment (start 143.2327 87.6323) (end 143.085 87.78) (width 0.2998) (layer "F.Cu") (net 1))
 (segment (start 137.2299 89.9184) (end 137.2299 89.2951) (width 0.4) (layer "F.Cu") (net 1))
 (segment (start 128.143 81.788) (end 128.143 82.9311) (width 0.4) (layer "F.Cu") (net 1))
 (segment (start 137.6225 87.8175) (end 137.585 87.78) (width 0.2998) (layer "F.Cu") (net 1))
 (segment (start 135.8893 90.6774) (end 136.4709 90.6774) (width 0.4) (layer "F.Cu") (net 1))
 (segment (start 128.143 82.9311) (end 135.8893 90.6774) (width 0.4) (layer "F.Cu") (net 1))
 (segment (start 137.6225 88.9025) (end 137.6225 87.8175) (width 0.2998) (layer "F.Cu") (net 1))
 (segment (start 136.4709 90.6774) (end 137.2299 89.9184) (width 0.4) (layer "F.Cu") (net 1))
 (segment (start 144.3584 86.8376) (end 144.0274 86.8376) (width 0.4) (layer "F.Cu") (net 1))
 (segment (start 137.535 88.99) (end 137.6225 88.9025) (width 0.2998) (layer "F.Cu") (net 1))
 (via (at 144.3584 86.8376) (size 0.8) (drill 0.4) (layers "F.Cu" "B.Cu") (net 1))
 (segment (start 151.0624 83.5155) (end 150.5397 82.9928) (width 0.4) (layer "B.Cu") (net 1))
 (segment (start 142.9576 88.8126) (end 143.135 88.99) (width 0.4) (layer "B.Cu") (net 1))
 (segment (start 151.0624 84.0278) (end 151.0624 83.5155) (width 0.4) (layer "B.Cu") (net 1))
 (segment (start 142.9576 88.0067) (end 142.9576 88.8126) (width 0.4) (layer "B.Cu") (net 1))
 (segment (start 144.3584 86.8376) (end 144.1267 86.8376) (width 0.4) (layer "B.Cu") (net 1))
 (segment (start 144.3584 86.8376) (end 148.2526 86.8376) (width 0.4) (layer "B.Cu") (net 1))
 (segment (start 144.1267 86.8376) (end 142.9576 88.0067) (width 0.4) (layer "B.Cu") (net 1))
 (segment (start 150.5397 82.9928) (end 143.5322 82.9928) (width 0.4) (layer "B.Cu") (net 1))
 (segment (start 143.5322 82.9928) (end 137.535 88.99) (width 0.4) (layer "B.Cu") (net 1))
 (segment (start 148.2526 86.8376) (end 151.0624 84.0278) (width 0.4) (layer "B.Cu") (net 1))
 (segment (start 141.085 82.538) (end 140.335 81.788) (width 0.3) (layer "F.Cu") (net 8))
 (segment (start 141.085 87.78) (end 141.085 82.538) (width 0.3) (layer "F.Cu") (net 8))
 (segment (start 142.085 84.102) (end 144.399 81.788) (width 0.3) (layer "F.Cu") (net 9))
 (segment (start 142.085 87.78) (end 142.085 84.102) (width 0.3) (layer "F.Cu") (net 9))
 (segment (start 142.585 87.0281) (end 147.8251 81.788) (width 0.3) (layer "F.Cu") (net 10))
 (segment (start 142.585 87.78) (end 142.585 87.0281) (width 0.3) (layer "F.Cu") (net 10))
 (segment (start 147.8251 81.788) (end 148.463 81.788) (width 0.3) (layer "F.Cu") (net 10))
 (segment (start 132.207 77.7264) (end 132.207 77.724) (width 0.3) (layer "F.Cu") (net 11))
 (segment (start 133.6946 79.214) (end 132.207 77.7264) (width 0.3) (layer "F.Cu") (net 11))
 (via (at 133.6946 79.214) (size 0.8) (drill 0.4) (layers "F.Cu" "B.Cu") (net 11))
 (segment (start 140.9733 91.5313) (end 142.735 89.7696) (width 0.3) (layer "B.Cu") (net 11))
 (segment (start 142.735 89.7696) (end 142.735 89.69) (width 0.3) (layer "B.Cu") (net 11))
 (segment (start 133.6946 89.7681) (end 135.4578 91.5313) (width 0.3) (layer "B.Cu") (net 11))
 (segment (start 135.4578 91.5313) (end 140.9733 91.5313) (width 0.3) (layer "B.Cu") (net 11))
 (segment (start 133.6946 79.214) (end 133.6946 89.7681) (width 0.3) (layer "B.Cu") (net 11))
 (segment (start 136.271 78.3589) (end 136.271 77.724) (width 0.3) (layer "F.Cu") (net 12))
 (segment (start 135.1039 79.526) (end 136.271 78.3589) (width 0.3) (layer "F.Cu") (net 12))
 (via (at 135.1039 79.526) (size 0.8) (drill 0.4) (layers "F.Cu" "B.Cu") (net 12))
 (segment (start 134.9721 79.6578) (end 134.9721 90.394) (width 0.3) (layer "B.Cu") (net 12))
 (segment (start 134.9721 90.394) (end 135.6559 91.0778) (width 0.3) (layer "B.Cu") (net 12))
 (segment (start 140.6196 91.0778) (end 141.935 89.7624) (width 0.3) (layer "B.Cu") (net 12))
 (segment (start 135.1039 79.526) (end 134.9721 79.6578) (width 0.3) (layer "B.Cu") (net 12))
 (segment (start 141.935 89.7624) (end 141.935 89.69) (width 0.3) (layer "B.Cu") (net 12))
 (segment (start 135.6559 91.0778) (end 140.6196 91.0778) (width 0.3) (layer "B.Cu") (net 12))
 (segment (start 140.335 78.078) (end 140.335 77.724) (width 0.3) (layer "F.Cu") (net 16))
 (segment (start 138.9865 79.4265) (end 140.335 78.078) (width 0.3) (layer "F.Cu") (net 16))
 (via (at 138.9865 79.4265) (size 0.8) (drill 0.4) (layers "F.Cu" "B.Cu") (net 16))
 (segment (start 135.8789 90.6032) (end 135.4642 90.1885) (width 0.3) (layer "B.Cu") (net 16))
 (segment (start 139.535 89.69) (end 139.535 89.7854) (width 0.3) (layer "B.Cu") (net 16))
 (segment (start 138.7172 90.6032) (end 135.8789 90.6032) (width 0.3) (layer "B.Cu") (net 16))
 (segment (start 135.4642 90.1885) (end 135.4642 82.9488) (width 0.3) (layer "B.Cu") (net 16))
 (segment (start 139.535 89.7854) (end 138.7172 90.6032) (width 0.3) (layer "B.Cu") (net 16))
 (segment (start 135.4642 82.9488) (end 138.9865 79.4265) (width 0.3) (layer "B.Cu") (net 16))
 (segment (start 150.3072 79.5682) (end 148.463 77.724) (width 0.3) (layer "F.Cu") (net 17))
 (segment (start 138.735 89.69) (end 138.735 89.7661) (width 0.3) (layer "F.Cu") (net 17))
 (segment (start 139.5554 90.5865) (end 144.8016 90.5865) (width 0.3) (layer "F.Cu") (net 17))
 (segment (start 145.3943 89.9938) (end 145.3943 87.4254) (width 0.3) (layer "F.Cu") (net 17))
 (segment (start 138.735 89.7661) (end 139.5554 90.5865) (width 0.3) (layer "F.Cu") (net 17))
 (segment (start 144.8016 90.5865) (end 145.3943 89.9938) (width 0.3) (layer "F.Cu") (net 17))
 (segment (start 150.3072 82.5125) (end 150.3072 79.5682) (width 0.3) (layer "F.Cu") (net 17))
 (segment (start 145.3943 87.4254) (end 150.3072 82.5125) (width 0.3) (layer "F.Cu") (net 17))
 (segment (start 145.8929 91.0461) (end 154.3565 82.5825) (width 0.3) (layer "F.Cu") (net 18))
 (segment (start 154.3565 82.5825) (end 154.3565 76.9802) (width 0.3) (layer "F.Cu") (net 18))
 (segment (start 139.1733 91.0461) (end 145.8929 91.0461) (width 0.3) (layer "F.Cu") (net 18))
 (segment (start 146.2235 75.8995) (end 144.399 77.724) (width 0.3) (layer "F.Cu") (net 18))
 (segment (start 137.935 89.8078) (end 139.1733 91.0461) (width 0.3) (layer "F.Cu") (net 18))
 (segment (start 154.3565 76.9802) (end 153.2758 75.8995) (width 0.3) (layer "F.Cu") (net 18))
 (segment (start 153.2758 75.8995) (end 146.2235 75.8995) (width 0.3) (layer "F.Cu") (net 18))
 (segment (start 137.935 89.69) (end 137.935 89.8078) (width 0.3) (layer "F.Cu") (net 18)))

